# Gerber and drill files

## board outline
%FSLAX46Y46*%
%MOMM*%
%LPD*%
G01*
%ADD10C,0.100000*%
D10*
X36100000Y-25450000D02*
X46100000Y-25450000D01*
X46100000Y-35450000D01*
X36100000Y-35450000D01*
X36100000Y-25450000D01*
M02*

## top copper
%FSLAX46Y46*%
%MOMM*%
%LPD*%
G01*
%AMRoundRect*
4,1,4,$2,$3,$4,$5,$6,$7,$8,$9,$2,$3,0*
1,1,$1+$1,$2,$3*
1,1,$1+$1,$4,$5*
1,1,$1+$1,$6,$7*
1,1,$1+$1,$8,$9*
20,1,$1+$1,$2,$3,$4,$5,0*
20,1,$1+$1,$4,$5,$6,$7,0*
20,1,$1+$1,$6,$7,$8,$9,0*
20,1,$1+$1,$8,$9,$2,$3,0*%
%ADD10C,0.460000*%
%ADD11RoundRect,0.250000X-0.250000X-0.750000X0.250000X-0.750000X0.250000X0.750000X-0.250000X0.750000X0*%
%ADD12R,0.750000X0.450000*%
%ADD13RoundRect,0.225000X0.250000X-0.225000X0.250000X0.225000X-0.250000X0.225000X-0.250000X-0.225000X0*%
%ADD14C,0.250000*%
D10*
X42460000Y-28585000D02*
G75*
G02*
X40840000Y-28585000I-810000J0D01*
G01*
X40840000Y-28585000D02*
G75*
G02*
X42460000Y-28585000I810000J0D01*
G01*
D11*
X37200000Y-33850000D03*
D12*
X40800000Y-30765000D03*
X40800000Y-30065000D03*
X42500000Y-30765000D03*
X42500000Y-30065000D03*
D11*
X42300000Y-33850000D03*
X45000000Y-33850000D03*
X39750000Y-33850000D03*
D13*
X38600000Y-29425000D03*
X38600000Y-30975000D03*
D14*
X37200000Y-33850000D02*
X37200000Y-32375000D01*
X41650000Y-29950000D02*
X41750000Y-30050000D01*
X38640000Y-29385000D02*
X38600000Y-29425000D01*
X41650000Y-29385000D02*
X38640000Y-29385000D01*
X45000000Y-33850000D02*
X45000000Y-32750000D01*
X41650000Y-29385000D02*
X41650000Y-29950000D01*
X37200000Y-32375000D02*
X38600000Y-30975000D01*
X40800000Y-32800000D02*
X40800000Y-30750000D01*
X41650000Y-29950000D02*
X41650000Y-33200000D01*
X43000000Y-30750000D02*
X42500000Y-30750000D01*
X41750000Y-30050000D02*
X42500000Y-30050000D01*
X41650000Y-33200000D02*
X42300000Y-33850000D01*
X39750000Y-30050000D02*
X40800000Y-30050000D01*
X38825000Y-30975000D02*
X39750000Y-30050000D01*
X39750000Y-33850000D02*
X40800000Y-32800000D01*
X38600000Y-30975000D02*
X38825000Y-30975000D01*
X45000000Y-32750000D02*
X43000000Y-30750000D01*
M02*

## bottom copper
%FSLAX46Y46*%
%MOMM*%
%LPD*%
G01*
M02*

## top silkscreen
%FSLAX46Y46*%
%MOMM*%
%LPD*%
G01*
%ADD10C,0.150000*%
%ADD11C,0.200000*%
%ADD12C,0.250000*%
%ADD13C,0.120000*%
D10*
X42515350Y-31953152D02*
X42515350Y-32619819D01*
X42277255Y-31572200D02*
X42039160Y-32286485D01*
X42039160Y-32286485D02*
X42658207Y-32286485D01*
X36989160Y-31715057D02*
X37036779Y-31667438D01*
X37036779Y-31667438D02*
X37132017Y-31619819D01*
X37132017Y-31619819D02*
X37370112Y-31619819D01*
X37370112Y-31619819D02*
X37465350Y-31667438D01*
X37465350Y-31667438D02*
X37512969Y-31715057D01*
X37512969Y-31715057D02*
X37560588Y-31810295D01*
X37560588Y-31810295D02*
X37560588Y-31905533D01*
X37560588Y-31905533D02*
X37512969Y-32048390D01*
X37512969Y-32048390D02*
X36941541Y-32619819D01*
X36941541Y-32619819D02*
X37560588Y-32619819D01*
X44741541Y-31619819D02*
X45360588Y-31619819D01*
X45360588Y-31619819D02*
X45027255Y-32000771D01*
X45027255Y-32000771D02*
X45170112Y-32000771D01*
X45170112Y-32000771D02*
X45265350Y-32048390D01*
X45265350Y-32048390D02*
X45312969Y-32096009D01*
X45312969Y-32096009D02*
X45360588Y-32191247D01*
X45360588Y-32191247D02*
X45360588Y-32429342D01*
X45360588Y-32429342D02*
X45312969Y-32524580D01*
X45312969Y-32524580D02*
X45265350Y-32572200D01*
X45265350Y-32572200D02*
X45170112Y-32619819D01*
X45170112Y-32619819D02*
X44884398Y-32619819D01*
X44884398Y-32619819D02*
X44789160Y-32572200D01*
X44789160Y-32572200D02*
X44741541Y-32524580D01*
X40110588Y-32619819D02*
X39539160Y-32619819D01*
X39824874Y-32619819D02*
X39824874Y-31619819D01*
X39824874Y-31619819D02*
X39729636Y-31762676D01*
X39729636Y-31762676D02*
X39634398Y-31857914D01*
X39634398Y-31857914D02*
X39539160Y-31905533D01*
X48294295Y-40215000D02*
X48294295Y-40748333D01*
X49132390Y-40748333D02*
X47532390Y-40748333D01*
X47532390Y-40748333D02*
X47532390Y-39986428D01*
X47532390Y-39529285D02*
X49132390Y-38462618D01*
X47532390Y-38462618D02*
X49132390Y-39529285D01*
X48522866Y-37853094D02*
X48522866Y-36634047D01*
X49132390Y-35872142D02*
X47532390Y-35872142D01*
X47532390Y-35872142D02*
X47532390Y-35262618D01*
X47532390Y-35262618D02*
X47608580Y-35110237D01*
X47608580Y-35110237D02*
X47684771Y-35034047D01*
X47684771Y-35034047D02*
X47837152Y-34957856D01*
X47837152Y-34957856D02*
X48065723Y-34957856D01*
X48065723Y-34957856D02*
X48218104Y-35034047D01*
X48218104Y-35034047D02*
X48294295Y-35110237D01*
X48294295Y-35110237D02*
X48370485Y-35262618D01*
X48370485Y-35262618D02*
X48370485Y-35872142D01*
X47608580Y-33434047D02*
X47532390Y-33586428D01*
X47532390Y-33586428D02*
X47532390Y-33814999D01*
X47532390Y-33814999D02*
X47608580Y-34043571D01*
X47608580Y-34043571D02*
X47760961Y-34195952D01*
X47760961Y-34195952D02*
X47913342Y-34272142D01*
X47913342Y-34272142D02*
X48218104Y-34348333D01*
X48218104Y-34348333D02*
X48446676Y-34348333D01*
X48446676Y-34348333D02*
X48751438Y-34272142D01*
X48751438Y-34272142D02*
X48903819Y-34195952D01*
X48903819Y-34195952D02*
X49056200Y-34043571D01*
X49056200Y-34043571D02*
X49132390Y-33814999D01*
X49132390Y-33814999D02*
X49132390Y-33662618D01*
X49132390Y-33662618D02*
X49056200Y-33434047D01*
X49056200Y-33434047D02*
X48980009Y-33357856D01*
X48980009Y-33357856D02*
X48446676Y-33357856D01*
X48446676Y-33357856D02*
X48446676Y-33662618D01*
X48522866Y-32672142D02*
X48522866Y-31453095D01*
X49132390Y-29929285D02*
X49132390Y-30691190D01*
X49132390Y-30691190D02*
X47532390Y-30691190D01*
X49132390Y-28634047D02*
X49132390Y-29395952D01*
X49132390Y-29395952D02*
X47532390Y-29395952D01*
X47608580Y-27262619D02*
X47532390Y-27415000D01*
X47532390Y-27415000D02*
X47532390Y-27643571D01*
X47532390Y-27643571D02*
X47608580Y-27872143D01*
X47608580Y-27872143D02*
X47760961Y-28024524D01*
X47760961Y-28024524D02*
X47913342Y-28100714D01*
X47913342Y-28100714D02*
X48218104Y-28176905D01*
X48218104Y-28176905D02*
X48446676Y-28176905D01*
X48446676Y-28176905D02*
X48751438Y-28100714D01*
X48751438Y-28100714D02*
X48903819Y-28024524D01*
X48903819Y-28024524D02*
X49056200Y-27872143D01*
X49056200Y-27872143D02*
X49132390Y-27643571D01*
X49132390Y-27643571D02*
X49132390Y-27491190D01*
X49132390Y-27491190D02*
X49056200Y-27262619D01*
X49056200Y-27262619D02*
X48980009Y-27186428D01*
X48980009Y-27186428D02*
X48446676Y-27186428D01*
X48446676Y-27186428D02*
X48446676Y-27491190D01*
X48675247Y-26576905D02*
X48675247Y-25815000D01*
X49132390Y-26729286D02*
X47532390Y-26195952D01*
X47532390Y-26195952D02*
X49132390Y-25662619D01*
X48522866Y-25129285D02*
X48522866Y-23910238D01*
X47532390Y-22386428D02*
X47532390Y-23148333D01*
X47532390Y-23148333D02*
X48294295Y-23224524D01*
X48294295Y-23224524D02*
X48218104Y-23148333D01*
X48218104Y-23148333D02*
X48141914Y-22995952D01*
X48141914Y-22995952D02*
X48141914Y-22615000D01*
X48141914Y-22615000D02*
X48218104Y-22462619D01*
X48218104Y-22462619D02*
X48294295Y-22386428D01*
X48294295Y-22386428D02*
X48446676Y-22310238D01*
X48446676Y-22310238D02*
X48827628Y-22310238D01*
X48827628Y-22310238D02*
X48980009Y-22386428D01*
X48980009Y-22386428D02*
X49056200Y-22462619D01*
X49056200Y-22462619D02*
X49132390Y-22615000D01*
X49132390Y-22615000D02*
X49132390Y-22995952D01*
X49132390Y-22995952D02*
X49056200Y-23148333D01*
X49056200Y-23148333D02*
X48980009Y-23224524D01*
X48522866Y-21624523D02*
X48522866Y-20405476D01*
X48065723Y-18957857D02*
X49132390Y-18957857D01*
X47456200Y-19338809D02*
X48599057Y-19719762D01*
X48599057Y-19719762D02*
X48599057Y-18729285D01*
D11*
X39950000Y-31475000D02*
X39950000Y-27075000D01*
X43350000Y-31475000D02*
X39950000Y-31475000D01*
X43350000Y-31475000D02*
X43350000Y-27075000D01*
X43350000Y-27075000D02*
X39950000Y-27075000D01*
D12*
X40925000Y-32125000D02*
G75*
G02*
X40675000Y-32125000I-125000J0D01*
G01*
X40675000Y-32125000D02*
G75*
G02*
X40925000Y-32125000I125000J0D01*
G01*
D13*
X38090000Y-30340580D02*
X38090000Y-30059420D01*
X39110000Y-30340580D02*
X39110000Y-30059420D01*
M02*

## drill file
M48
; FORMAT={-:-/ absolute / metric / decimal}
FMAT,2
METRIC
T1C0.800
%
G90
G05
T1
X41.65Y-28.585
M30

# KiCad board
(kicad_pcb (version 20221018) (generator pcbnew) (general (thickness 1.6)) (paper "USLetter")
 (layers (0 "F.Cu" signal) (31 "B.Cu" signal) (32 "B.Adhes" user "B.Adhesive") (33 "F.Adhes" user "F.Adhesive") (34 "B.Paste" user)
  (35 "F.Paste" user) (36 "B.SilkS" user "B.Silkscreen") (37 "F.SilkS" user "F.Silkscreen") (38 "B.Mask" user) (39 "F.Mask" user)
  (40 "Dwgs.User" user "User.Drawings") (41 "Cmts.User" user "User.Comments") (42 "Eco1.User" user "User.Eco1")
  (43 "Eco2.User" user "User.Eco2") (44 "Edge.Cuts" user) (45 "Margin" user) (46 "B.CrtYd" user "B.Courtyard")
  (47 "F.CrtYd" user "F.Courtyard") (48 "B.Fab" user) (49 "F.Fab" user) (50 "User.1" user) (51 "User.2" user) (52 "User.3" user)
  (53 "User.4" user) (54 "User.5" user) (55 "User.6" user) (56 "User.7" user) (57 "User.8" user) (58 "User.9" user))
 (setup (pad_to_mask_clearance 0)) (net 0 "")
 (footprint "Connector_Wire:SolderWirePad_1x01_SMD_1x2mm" (layer "F.Cu") (at 37.2 33.85)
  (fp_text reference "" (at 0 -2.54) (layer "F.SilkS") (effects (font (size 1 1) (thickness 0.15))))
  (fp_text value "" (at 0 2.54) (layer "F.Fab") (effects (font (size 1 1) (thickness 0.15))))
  (pad "2" smd roundrect (at 0 0) (size 1 2) (layers "F.Cu" "F.Paste" "F.Mask") (roundrect_rratio 0.25)))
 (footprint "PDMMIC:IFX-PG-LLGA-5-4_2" (layer "F.Cu") (at 41.65 29.675 90)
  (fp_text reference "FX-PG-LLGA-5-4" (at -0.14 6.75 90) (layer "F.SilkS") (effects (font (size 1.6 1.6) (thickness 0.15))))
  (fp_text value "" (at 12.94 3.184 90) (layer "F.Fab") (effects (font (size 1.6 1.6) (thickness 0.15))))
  (fp_circle (center 1.09 0) (end 1.9 0) (stroke (width 0.46) (type solid)) (fill none) (layer "F.Cu"))
  (fp_line (start -1.8 -1.7) (end 2.6 -1.7) (stroke (width 0.2) (type solid)) (layer "F.SilkS"))
  (fp_line (start -1.8 1.7) (end -1.8 -1.7) (stroke (width 0.2) (type solid)) (layer "F.SilkS"))
  (fp_line (start -1.8 1.7) (end 2.6 1.7) (stroke (width 0.2) (type solid)) (layer "F.SilkS"))
  (fp_line (start 2.6 1.7) (end 2.6 -1.7) (stroke (width 0.2) (type solid)) (layer "F.SilkS"))
  (fp_circle (center -2.45 -0.85) (end -2.325 -0.85) (stroke (width 0.25) (type solid)) (fill none) (layer "F.SilkS"))
  (pad "" np_thru_hole circle (at 1.09 0 90) (size 0.8 0.8) (drill 0.8) (layers "F&B.Cu" "*.Mask"))
  (pad "1" smd rect (at -1.09 -0.85 90) (size 0.45 0.75) (layers "F.Cu" "F.Mask") (solder_mask_margin 0.102))
  (pad "2" smd rect (at -0.39 -0.85 90) (size 0.45 0.75) (layers "F.Cu" "F.Mask") (solder_mask_margin 0.102))
  (pad "3" smd rect (at -1.09 0.85 90) (size 0.45 0.75) (layers "F.Cu" "F.Mask") (solder_mask_margin 0.102))
  (pad "4" smd rect (at -0.39 0.85 90) (size 0.45 0.75) (layers "F.Cu" "F.Mask") (solder_mask_margin 0.102)))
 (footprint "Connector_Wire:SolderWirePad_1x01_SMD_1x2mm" (layer "F.Cu") (at 42.3 33.85)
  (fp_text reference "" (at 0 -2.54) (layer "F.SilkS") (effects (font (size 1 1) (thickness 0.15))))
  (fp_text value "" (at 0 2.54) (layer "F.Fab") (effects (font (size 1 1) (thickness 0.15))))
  (pad "4" smd roundrect (at 0 0) (size 1 2) (layers "F.Cu" "F.Paste" "F.Mask") (roundrect_rratio 0.25)))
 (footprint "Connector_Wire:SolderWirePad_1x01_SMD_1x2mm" (layer "F.Cu") (at 45 33.85)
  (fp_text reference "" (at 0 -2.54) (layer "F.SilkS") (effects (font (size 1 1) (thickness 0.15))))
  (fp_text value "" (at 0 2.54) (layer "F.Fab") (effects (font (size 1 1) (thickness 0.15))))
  (pad "3" smd roundrect (at 0 0) (size 1 2) (layers "F.Cu" "F.Paste" "F.Mask") (roundrect_rratio 0.25)))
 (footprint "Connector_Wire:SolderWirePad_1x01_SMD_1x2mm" (layer "F.Cu") (at 39.75 33.85)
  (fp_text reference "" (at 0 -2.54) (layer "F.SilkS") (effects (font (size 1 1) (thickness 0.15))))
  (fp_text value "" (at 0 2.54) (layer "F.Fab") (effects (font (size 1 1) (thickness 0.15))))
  (pad "1" smd roundrect (at 0 0) (size 1 2) (layers "F.Cu" "F.Paste" "F.Mask") (roundrect_rratio 0.25)))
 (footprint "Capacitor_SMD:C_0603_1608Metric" (layer "F.Cu") (at 38.6 30.2 90)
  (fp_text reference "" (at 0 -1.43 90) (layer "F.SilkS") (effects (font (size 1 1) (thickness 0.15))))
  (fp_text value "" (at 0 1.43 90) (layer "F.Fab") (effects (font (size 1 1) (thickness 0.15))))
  (fp_line (start -0.14058 -0.51) (end 0.14058 -0.51) (stroke (width 0.12) (type solid)) (layer "F.SilkS"))
  (fp_line (start -0.14058 0.51) (end 0.14058 0.51) (stroke (width 0.12) (type solid)) (layer "F.SilkS"))
  (pad "1" smd roundrect (at 0.775 0 90) (size 0.9 0.95) (layers "F.Cu" "F.Paste" "F.Mask") (roundrect_rratio 0.25))
  (pad "2" smd roundrect (at -0.775 0 90) (size 0.9 0.95) (layers "F.Cu" "F.Paste" "F.Mask") (roundrect_rratio 0.25)))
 (gr_rect (start 36.1 25.45) (end 46.1 35.45) (stroke (width 0.1) (type default)) (fill none) (layer "Edge.Cuts"))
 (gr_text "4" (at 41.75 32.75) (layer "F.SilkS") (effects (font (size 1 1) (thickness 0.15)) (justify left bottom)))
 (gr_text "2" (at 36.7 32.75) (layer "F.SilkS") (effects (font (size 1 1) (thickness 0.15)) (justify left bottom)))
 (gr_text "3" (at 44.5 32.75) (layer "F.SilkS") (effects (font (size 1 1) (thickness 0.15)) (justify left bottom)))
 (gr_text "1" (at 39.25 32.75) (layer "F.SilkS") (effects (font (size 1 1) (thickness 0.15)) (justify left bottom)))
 (segment (start 37.2 33.85) (end 37.2 32.375) (width 0.25) (layer "F.Cu") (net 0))
 (segment (start 41.65 29.95) (end 41.75 30.05) (width 0.25) (layer "F.Cu") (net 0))
 (segment (start 38.64 29.385) (end 38.6 29.425) (width 0.25) (layer "F.Cu") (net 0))
 (segment (start 41.65 29.385) (end 38.64 29.385) (width 0.25) (layer "F.Cu") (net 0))
 (segment (start 45 33.85) (end 45 32.75) (width 0.25) (layer "F.Cu") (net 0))
 (segment (start 41.65 29.385) (end 41.65 29.95) (width 0.25) (layer "F.Cu") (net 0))
 (segment (start 37.2 32.375) (end 38.6 30.975) (width 0.25) (layer "F.Cu") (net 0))
 (segment (start 40.8 32.8) (end 40.8 30.75) (width 0.25) (layer "F.Cu") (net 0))
 (segment (start 41.65 29.95) (end 41.65 33.2) (width 0.25) (layer "F.Cu") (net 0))
 (segment (start 43 30.75) (end 42.5 30.75) (width 0.25) (layer "F.Cu") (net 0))
 (segment (start 41.75 30.05) (end 42.5 30.05) (width 0.25) (layer "F.Cu") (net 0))
 (segment (start 41.65 33.2) (end 42.3 33.85) (width 0.25) (layer "F.Cu") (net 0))
 (segment (start 39.75 30.05) (end 40.8 30.05) (width 0.25) (layer "F.Cu") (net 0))
 (segment (start 38.825 30.975) (end 39.75 30.05) (width 0.25) (layer "F.Cu") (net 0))
 (segment (start 39.75 33.85) (end 40.8 32.8) (width 0.25) (layer "F.Cu") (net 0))
 (segment (start 38.6 30.975) (end 38.825 30.975) (width 0.25) (layer "F.Cu") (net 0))
 (segment (start 45 32.75) (end 43 30.75) (width 0.25) (layer "F.Cu") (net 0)))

